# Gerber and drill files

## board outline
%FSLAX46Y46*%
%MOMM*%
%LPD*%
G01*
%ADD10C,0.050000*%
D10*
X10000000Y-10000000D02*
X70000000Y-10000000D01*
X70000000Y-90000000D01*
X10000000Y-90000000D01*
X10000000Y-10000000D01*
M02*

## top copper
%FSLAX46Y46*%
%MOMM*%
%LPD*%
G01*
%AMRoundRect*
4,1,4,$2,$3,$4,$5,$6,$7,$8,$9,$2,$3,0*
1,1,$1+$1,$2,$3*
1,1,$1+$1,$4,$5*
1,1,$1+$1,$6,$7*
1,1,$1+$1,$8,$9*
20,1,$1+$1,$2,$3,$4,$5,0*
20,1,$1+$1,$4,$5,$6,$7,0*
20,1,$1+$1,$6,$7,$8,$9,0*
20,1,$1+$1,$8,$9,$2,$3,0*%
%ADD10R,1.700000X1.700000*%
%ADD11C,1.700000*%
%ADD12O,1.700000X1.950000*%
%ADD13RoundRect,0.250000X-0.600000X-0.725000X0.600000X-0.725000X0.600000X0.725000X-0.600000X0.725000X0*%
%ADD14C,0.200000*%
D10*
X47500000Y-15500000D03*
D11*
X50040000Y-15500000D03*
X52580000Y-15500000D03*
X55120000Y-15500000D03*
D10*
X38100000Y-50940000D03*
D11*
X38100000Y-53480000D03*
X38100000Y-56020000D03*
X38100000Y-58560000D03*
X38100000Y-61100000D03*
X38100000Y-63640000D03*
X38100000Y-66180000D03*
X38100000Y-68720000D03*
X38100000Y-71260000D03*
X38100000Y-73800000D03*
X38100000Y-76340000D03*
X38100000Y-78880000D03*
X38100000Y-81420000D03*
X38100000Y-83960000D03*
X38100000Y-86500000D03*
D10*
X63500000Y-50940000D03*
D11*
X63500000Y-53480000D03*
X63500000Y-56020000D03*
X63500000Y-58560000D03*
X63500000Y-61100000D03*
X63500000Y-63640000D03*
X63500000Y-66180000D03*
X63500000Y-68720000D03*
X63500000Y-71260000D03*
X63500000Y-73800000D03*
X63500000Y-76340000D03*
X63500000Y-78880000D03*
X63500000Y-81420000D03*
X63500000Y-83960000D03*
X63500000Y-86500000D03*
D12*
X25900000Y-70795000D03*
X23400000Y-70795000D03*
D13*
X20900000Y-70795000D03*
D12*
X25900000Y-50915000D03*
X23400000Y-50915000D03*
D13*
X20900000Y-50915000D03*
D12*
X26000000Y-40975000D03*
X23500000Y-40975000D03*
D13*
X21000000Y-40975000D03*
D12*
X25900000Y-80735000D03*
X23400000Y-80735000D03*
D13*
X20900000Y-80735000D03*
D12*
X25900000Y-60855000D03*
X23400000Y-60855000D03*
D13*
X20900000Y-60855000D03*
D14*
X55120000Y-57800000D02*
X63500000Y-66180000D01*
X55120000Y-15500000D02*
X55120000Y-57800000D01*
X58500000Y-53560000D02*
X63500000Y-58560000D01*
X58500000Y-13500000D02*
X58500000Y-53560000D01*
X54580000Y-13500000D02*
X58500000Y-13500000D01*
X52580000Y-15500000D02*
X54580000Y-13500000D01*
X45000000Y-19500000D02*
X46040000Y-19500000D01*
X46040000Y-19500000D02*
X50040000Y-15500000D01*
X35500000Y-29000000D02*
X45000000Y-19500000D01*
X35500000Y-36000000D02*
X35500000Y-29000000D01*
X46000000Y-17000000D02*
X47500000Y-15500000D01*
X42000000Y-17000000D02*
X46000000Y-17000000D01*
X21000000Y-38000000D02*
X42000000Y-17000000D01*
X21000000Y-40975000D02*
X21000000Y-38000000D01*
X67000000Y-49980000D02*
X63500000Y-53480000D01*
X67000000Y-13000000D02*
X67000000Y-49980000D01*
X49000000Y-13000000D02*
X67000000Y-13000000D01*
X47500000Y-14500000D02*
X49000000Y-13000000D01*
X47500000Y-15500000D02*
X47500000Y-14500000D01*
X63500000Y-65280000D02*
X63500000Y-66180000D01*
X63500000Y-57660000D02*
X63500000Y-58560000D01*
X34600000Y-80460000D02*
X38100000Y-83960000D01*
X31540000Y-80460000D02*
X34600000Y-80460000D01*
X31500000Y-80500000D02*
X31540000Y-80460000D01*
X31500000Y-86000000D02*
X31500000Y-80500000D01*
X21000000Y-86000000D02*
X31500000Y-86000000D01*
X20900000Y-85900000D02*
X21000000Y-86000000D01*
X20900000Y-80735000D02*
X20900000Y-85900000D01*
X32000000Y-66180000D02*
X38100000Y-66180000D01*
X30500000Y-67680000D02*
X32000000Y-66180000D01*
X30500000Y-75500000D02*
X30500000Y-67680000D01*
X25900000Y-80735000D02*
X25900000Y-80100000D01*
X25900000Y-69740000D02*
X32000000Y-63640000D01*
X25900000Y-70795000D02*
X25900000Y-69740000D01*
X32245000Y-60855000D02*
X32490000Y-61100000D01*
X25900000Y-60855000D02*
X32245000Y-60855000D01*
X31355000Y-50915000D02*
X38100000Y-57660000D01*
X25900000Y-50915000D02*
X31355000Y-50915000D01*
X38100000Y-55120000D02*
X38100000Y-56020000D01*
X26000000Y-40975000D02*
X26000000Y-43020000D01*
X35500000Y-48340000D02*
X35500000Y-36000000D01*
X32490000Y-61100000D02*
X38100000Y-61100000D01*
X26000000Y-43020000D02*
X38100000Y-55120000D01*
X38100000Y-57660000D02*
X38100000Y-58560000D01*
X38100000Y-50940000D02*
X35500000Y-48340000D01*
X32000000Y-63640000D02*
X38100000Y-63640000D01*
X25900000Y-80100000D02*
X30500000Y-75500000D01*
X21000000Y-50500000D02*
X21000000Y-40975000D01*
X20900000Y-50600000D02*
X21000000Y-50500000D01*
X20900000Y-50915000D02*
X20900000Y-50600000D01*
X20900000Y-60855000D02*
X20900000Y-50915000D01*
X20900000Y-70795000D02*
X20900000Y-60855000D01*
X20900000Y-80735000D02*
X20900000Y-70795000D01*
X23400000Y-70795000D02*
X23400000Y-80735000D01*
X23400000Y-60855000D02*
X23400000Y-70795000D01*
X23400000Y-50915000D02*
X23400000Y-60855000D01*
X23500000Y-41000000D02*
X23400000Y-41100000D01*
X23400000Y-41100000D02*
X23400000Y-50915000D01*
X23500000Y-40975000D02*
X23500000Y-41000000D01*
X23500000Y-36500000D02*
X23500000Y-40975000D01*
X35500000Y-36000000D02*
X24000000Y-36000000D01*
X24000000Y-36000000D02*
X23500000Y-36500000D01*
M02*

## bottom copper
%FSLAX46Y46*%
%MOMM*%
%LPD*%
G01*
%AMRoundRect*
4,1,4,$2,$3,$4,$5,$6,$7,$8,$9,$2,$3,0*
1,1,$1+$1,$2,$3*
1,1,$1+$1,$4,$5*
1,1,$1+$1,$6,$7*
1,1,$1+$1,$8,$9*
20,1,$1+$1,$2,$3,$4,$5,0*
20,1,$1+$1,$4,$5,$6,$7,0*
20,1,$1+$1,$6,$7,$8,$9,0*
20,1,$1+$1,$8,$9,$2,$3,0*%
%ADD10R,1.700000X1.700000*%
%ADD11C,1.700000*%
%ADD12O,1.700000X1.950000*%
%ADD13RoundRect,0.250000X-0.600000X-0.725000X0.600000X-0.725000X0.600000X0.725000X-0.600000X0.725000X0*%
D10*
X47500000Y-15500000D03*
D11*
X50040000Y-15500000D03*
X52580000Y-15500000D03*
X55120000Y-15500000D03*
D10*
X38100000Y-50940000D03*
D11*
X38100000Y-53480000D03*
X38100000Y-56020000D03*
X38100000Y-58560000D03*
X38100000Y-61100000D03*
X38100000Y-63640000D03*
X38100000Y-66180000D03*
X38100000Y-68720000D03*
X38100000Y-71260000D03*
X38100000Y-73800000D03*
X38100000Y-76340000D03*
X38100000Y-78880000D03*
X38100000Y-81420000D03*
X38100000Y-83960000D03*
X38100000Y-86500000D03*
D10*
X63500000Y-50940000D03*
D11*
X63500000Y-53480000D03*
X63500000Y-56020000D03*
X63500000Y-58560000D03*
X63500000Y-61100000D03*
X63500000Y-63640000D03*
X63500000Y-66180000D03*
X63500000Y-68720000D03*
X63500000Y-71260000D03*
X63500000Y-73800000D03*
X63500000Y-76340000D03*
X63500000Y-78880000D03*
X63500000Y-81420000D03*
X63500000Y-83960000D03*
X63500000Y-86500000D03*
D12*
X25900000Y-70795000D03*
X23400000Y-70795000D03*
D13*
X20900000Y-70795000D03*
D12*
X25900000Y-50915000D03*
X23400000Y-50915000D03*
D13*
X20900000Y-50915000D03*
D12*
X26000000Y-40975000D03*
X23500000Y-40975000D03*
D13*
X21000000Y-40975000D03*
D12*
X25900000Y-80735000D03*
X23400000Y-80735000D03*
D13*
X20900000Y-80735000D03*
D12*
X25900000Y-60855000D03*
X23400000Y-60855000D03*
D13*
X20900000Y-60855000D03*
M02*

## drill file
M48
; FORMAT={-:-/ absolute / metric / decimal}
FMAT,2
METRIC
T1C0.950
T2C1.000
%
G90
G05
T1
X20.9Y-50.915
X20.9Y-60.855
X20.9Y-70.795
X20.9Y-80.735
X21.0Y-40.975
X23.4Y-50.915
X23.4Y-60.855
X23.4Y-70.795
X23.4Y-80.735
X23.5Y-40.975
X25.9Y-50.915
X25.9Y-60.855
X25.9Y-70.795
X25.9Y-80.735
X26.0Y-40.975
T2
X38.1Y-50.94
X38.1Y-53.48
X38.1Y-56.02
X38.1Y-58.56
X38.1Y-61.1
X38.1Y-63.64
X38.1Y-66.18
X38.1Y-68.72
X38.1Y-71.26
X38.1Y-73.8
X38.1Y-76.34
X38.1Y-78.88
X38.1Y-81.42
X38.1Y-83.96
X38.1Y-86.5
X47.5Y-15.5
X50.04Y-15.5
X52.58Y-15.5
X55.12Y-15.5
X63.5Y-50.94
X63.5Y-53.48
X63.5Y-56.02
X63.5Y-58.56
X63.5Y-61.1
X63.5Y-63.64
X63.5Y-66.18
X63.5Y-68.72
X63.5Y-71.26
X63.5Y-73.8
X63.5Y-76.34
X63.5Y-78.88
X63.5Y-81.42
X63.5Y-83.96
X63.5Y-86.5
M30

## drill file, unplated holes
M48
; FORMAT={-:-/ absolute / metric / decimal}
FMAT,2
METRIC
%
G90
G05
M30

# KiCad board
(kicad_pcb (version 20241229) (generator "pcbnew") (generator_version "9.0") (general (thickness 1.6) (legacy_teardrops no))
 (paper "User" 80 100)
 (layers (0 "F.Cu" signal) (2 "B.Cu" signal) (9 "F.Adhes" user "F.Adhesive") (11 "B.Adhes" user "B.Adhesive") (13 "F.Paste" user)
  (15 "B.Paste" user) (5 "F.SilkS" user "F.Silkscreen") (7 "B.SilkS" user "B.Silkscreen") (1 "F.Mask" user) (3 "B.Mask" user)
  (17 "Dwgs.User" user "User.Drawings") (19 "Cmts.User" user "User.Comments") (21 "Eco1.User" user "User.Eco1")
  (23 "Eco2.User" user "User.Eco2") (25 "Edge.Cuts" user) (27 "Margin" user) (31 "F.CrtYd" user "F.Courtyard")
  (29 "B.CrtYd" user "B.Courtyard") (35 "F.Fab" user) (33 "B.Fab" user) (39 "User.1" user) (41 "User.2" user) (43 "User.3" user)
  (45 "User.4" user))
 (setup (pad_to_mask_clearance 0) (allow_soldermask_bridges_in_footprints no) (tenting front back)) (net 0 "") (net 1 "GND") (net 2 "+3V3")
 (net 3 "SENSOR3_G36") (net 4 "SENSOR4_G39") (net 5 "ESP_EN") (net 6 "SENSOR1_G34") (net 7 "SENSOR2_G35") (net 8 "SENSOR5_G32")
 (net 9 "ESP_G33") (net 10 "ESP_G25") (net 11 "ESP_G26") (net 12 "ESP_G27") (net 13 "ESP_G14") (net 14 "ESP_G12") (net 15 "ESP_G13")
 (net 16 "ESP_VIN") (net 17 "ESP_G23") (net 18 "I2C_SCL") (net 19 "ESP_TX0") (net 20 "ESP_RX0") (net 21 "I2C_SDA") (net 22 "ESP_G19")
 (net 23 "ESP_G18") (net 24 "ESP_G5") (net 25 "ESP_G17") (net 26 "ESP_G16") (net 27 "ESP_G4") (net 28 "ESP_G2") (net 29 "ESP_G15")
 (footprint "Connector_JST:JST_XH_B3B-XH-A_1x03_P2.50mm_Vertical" (layer "F.Cu") (at 21 40.975)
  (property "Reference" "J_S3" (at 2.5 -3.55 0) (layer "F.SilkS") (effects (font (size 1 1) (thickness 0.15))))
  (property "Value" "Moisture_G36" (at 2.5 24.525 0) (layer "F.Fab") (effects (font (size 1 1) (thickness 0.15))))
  (pad "1" thru_hole roundrect (at 0 0) (size 1.7 1.95) (drill 0.95) (layers "*.Cu" "*.Mask") (remove_unused_layers no)
   (roundrect_rratio 0.147059) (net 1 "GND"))
  (pad "2" thru_hole oval (at 2.5 0) (size 1.7 1.95) (drill 0.95) (layers "*.Cu" "*.Mask") (remove_unused_layers no) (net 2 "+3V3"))
  (pad "3" thru_hole oval (at 5 0) (size 1.7 1.95) (drill 0.95) (layers "*.Cu" "*.Mask") (remove_unused_layers no) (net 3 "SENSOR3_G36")))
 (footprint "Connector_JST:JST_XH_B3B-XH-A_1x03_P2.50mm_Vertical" (layer "F.Cu") (at 20.9 50.915)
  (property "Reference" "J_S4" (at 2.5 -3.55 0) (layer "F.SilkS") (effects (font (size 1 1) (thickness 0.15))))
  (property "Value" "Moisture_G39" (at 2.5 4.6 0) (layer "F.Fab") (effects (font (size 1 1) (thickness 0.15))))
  (pad "1" thru_hole roundrect (at 0 0) (size 1.7 1.95) (drill 0.95) (layers "*.Cu" "*.Mask") (remove_unused_layers no)
   (roundrect_rratio 0.147059) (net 1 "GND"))
  (pad "2" thru_hole oval (at 2.5 0) (size 1.7 1.95) (drill 0.95) (layers "*.Cu" "*.Mask") (remove_unused_layers no) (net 2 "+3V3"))
  (pad "3" thru_hole oval (at 5 0) (size 1.7 1.95) (drill 0.95) (layers "*.Cu" "*.Mask") (remove_unused_layers no) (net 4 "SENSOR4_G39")))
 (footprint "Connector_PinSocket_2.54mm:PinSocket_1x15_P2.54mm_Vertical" (layer "F.Cu") (at 38.1 50.94)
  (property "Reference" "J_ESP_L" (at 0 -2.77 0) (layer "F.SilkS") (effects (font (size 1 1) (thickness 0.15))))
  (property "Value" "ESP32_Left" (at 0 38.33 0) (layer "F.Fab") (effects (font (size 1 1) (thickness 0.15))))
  (pad "1" thru_hole rect (at 0 0) (size 1.7 1.7) (drill 1) (layers "*.Cu" "*.Mask") (remove_unused_layers no) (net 2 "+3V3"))
  (pad "2" thru_hole circle (at 0 2.54) (size 1.7 1.7) (drill 1) (layers "*.Cu" "*.Mask") (remove_unused_layers no) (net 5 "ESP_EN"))
  (pad "3" thru_hole circle (at 0 5.08) (size 1.7 1.7) (drill 1) (layers "*.Cu" "*.Mask") (remove_unused_layers no) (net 3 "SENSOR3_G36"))
  (pad "4" thru_hole circle (at 0 7.62) (size 1.7 1.7) (drill 1) (layers "*.Cu" "*.Mask") (remove_unused_layers no) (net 4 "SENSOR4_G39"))
  (pad "5" thru_hole circle (at 0 10.16) (size 1.7 1.7) (drill 1) (layers "*.Cu" "*.Mask") (remove_unused_layers no) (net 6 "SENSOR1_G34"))
  (pad "6" thru_hole circle (at 0 12.7) (size 1.7 1.7) (drill 1) (layers "*.Cu" "*.Mask") (remove_unused_layers no) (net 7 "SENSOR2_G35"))
  (pad "7" thru_hole circle (at 0 15.24) (size 1.7 1.7) (drill 1) (layers "*.Cu" "*.Mask") (remove_unused_layers no) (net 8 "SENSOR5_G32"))
  (pad "8" thru_hole circle (at 0 17.78) (size 1.7 1.7) (drill 1) (layers "*.Cu" "*.Mask") (remove_unused_layers no) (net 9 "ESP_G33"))
  (pad "9" thru_hole circle (at 0 20.32) (size 1.7 1.7) (drill 1) (layers "*.Cu" "*.Mask") (remove_unused_layers no) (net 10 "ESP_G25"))
  (pad "10" thru_hole circle (at 0 22.86) (size 1.7 1.7) (drill 1) (layers "*.Cu" "*.Mask") (remove_unused_layers no) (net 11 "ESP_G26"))
  (pad "11" thru_hole circle (at 0 25.4) (size 1.7 1.7) (drill 1) (layers "*.Cu" "*.Mask") (remove_unused_layers no) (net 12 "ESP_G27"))
  (pad "12" thru_hole circle (at 0 27.94) (size 1.7 1.7) (drill 1) (layers "*.Cu" "*.Mask") (remove_unused_layers no) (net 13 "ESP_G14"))
  (pad "13" thru_hole circle (at 0 30.48) (size 1.7 1.7) (drill 1) (layers "*.Cu" "*.Mask") (remove_unused_layers no) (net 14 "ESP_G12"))
  (pad "14" thru_hole circle (at 0 33.02) (size 1.7 1.7) (drill 1) (layers "*.Cu" "*.Mask") (remove_unused_layers no) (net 1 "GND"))
  (pad "15" thru_hole circle (at 0 35.56) (size 1.7 1.7) (drill 1) (layers "*.Cu" "*.Mask") (remove_unused_layers no) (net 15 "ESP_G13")))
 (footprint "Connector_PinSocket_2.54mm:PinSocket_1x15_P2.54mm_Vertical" (layer "F.Cu") (at 63.5 50.94)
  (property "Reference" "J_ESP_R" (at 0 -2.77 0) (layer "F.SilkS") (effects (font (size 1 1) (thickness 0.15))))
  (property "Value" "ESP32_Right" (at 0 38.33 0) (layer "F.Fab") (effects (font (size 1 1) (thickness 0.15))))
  (pad "1" thru_hole rect (at 0 0) (size 1.7 1.7) (drill 1) (layers "*.Cu" "*.Mask") (remove_unused_layers no) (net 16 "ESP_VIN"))
  (pad "2" thru_hole circle (at 0 2.54) (size 1.7 1.7) (drill 1) (layers "*.Cu" "*.Mask") (remove_unused_layers no) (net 1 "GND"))
  (pad "3" thru_hole circle (at 0 5.08) (size 1.7 1.7) (drill 1) (layers "*.Cu" "*.Mask") (remove_unused_layers no) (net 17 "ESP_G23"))
  (pad "4" thru_hole circle (at 0 7.62) (size 1.7 1.7) (drill 1) (layers "*.Cu" "*.Mask") (remove_unused_layers no) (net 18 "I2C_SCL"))
  (pad "5" thru_hole circle (at 0 10.16) (size 1.7 1.7) (drill 1) (layers "*.Cu" "*.Mask") (remove_unused_layers no) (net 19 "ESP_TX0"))
  (pad "6" thru_hole circle (at 0 12.7) (size 1.7 1.7) (drill 1) (layers "*.Cu" "*.Mask") (remove_unused_layers no) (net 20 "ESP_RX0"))
  (pad "7" thru_hole circle (at 0 15.24) (size 1.7 1.7) (drill 1) (layers "*.Cu" "*.Mask") (remove_unused_layers no) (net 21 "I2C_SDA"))
  (pad "8" thru_hole circle (at 0 17.78) (size 1.7 1.7) (drill 1) (layers "*.Cu" "*.Mask") (remove_unused_layers no) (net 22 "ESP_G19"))
  (pad "9" thru_hole circle (at 0 20.32) (size 1.7 1.7) (drill 1) (layers "*.Cu" "*.Mask") (remove_unused_layers no) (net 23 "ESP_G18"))
  (pad "10" thru_hole circle (at 0 22.86) (size 1.7 1.7) (drill 1) (layers "*.Cu" "*.Mask") (remove_unused_layers no) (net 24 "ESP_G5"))
  (pad "11" thru_hole circle (at 0 25.4) (size 1.7 1.7) (drill 1) (layers "*.Cu" "*.Mask") (remove_unused_layers no) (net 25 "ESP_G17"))
  (pad "12" thru_hole circle (at 0 27.94) (size 1.7 1.7) (drill 1) (layers "*.Cu" "*.Mask") (remove_unused_layers no) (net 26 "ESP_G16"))
  (pad "13" thru_hole circle (at 0 30.48) (size 1.7 1.7) (drill 1) (layers "*.Cu" "*.Mask") (remove_unused_layers no) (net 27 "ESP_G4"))
  (pad "14" thru_hole circle (at 0 33.02) (size 1.7 1.7) (drill 1) (layers "*.Cu" "*.Mask") (remove_unused_layers no) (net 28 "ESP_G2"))
  (pad "15" thru_hole circle (at 0 35.56) (size 1.7 1.7) (drill 1) (layers "*.Cu" "*.Mask") (remove_unused_layers no) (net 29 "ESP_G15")))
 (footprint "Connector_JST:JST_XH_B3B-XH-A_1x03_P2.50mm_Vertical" (layer "F.Cu") (at 20.9 80.735)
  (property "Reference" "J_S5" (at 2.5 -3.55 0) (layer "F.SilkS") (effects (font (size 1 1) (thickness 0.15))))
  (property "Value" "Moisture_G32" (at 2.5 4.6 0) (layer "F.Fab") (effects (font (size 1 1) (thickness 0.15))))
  (pad "1" thru_hole roundrect (at 0 0) (size 1.7 1.95) (drill 0.95) (layers "*.Cu" "*.Mask") (remove_unused_layers no)
   (roundrect_rratio 0.147059) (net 1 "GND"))
  (pad "2" thru_hole oval (at 2.5 0) (size 1.7 1.95) (drill 0.95) (layers "*.Cu" "*.Mask") (remove_unused_layers no) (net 2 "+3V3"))
  (pad "3" thru_hole oval (at 5 0) (size 1.7 1.95) (drill 0.95) (layers "*.Cu" "*.Mask") (remove_unused_layers no) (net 8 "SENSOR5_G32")))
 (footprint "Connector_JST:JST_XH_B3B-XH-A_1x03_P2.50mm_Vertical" (layer "F.Cu") (at 20.9 60.855)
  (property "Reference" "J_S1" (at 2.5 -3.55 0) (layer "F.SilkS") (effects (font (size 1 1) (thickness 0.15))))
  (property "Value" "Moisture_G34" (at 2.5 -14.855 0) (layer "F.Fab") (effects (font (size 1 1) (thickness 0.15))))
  (pad "1" thru_hole roundrect (at 0 0) (size 1.7 1.95) (drill 0.95) (layers "*.Cu" "*.Mask") (remove_unused_layers no)
   (roundrect_rratio 0.147059) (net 1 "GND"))
  (pad "2" thru_hole oval (at 2.5 0) (size 1.7 1.95) (drill 0.95) (layers "*.Cu" "*.Mask") (remove_unused_layers no) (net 2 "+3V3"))
  (pad "3" thru_hole oval (at 5 0) (size 1.7 1.95) (drill 0.95) (layers "*.Cu" "*.Mask") (remove_unused_layers no) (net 6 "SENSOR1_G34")))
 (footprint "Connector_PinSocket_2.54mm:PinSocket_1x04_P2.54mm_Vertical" (layer "F.Cu") (at 47.5 15.5 90)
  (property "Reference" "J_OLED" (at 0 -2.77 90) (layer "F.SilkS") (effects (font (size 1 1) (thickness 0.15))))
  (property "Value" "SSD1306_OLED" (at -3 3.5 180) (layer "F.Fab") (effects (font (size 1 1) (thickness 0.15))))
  (pad "1" thru_hole rect (at 0 0 90) (size 1.7 1.7) (drill 1) (layers "*.Cu" "*.Mask") (remove_unused_layers no) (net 1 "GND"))
  (pad "2" thru_hole circle (at 0 2.54 90) (size 1.7 1.7) (drill 1) (layers "*.Cu" "*.Mask") (remove_unused_layers no) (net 2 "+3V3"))
  (pad "3" thru_hole circle (at 0 5.08 90) (size 1.7 1.7) (drill 1) (layers "*.Cu" "*.Mask") (remove_unused_layers no) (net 18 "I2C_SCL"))
  (pad "4" thru_hole circle (at 0 7.62 90) (size 1.7 1.7) (drill 1) (layers "*.Cu" "*.Mask") (remove_unused_layers no) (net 21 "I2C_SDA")))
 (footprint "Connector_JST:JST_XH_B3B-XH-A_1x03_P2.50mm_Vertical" (layer "F.Cu") (at 20.9 70.795)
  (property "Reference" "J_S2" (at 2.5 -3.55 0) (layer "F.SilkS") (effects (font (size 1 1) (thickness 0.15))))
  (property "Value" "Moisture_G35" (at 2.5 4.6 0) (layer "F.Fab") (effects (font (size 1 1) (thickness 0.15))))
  (pad "1" thru_hole roundrect (at 0 0) (size 1.7 1.95) (drill 0.95) (layers "*.Cu" "*.Mask") (remove_unused_layers no)
   (roundrect_rratio 0.147059) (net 1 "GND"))
  (pad "2" thru_hole oval (at 2.5 0) (size 1.7 1.95) (drill 0.95) (layers "*.Cu" "*.Mask") (remove_unused_layers no) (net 2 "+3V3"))
  (pad "3" thru_hole oval (at 5 0) (size 1.7 1.95) (drill 0.95) (layers "*.Cu" "*.Mask") (remove_unused_layers no) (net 7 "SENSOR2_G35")))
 (gr_rect (start 10 10) (end 70 90) (stroke (width 0.05) (type default)) (fill no) (layer "Edge.Cuts"))
 (segment (start 31.54 80.46) (end 34.6 80.46) (width 0.2) (layer "F.Cu") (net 1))
 (segment (start 20.9 85.9) (end 21 86) (width 0.2) (layer "F.Cu") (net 1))
 (segment (start 67 13) (end 67 49.98) (width 0.2) (layer "F.Cu") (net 1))
 (segment (start 67 49.98) (end 63.5 53.48) (width 0.2) (layer "F.Cu") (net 1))
 (segment (start 20.9 80.735) (end 20.9 85.9) (width 0.2) (layer "F.Cu") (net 1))
 (segment (start 21 40.975) (end 21 38) (width 0.2) (layer "F.Cu") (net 1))
 (segment (start 20.9 60.855) (end 20.9 50.915) (width 0.2) (layer "F.Cu") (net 1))
 (segment (start 20.9 50.6) (end 21 50.5) (width 0.2) (layer "F.Cu") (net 1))
 (segment (start 20.9 70.795) (end 20.9 60.855) (width 0.2) (layer "F.Cu") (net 1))
 (segment (start 31.5 80.5) (end 31.54 80.46) (width 0.2) (layer "F.Cu") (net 1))
 (segment (start 42 17) (end 46 17) (width 0.2) (layer "F.Cu") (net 1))
 (segment (start 31.5 86) (end 31.5 80.5) (width 0.2) (layer "F.Cu") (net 1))
 (segment (start 21 38) (end 42 17) (width 0.2) (layer "F.Cu") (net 1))
 (segment (start 21 50.5) (end 21 40.975) (width 0.2) (layer "F.Cu") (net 1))
 (segment (start 46 17) (end 47.5 15.5) (width 0.2) (layer "F.Cu") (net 1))
 (segment (start 20.9 80.735) (end 20.9 70.795) (width 0.2) (layer "F.Cu") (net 1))
 (segment (start 47.5 14.5) (end 49 13) (width 0.2) (layer "F.Cu") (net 1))
 (segment (start 49 13) (end 67 13) (width 0.2) (layer "F.Cu") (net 1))
 (segment (start 20.9 50.915) (end 20.9 50.6) (width 0.2) (layer "F.Cu") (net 1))
 (segment (start 47.5 15.5) (end 47.5 14.5) (width 0.2) (layer "F.Cu") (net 1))
 (segment (start 21 86) (end 31.5 86) (width 0.2) (layer "F.Cu") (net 1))
 (segment (start 34.6 80.46) (end 38.1 83.96) (width 0.2) (layer "F.Cu") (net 1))
 (segment (start 35.5 29) (end 45 19.5) (width 0.2) (layer "F.Cu") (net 2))
 (segment (start 23.5 36.5) (end 23.5 40.975) (width 0.2) (layer "F.Cu") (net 2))
 (segment (start 23.4 50.915) (end 23.4 60.855) (width 0.2) (layer "F.Cu") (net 2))
 (segment (start 23.4 60.855) (end 23.4 70.795) (width 0.2) (layer "F.Cu") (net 2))
 (segment (start 24 36) (end 23.5 36.5) (width 0.2) (layer "F.Cu") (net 2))
 (segment (start 23.5 40.975) (end 23.5 41) (width 0.2) (layer "F.Cu") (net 2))
 (segment (start 23.4 70.795) (end 23.4 80.735) (width 0.2) (layer "F.Cu") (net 2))
 (segment (start 23.4 41.1) (end 23.4 50.915) (width 0.2) (layer "F.Cu") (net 2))
 (segment (start 35.5 36) (end 35.5 29) (width 0.2) (layer "F.Cu") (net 2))
 (segment (start 35.5 48.34) (end 35.5 36) (width 0.2) (layer "F.Cu") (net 2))
 (segment (start 35.5 36) (end 24 36) (width 0.2) (layer "F.Cu") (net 2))
 (segment (start 45 19.5) (end 46.04 19.5) (width 0.2) (layer "F.Cu") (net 2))
 (segment (start 46.04 19.5) (end 50.04 15.5) (width 0.2) (layer "F.Cu") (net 2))
 (segment (start 38.1 50.94) (end 35.5 48.34) (width 0.2) (layer "F.Cu") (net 2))
 (segment (start 23.5 41) (end 23.4 41.1) (width 0.2) (layer "F.Cu") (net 2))
 (segment (start 31.355 50.915) (end 38.1 57.66) (width 0.2) (layer "F.Cu") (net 4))
 (segment (start 25.9 50.915) (end 31.355 50.915) (width 0.2) (layer "F.Cu") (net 4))
 (segment (start 38.1 57.66) (end 38.1 58.56) (width 0.2) (layer "F.Cu") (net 4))
 (segment (start 38.1 55.12) (end 38.1 56.02) (width 0.2) (layer "F.Cu") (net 3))
 (segment (start 26 43.02) (end 38.1 55.12) (width 0.2) (layer "F.Cu") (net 3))
 (segment (start 26 40.975) (end 26 43.02) (width 0.2) (layer "F.Cu") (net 3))
 (segment (start 25.9 80.1) (end 30.5 75.5) (width 0.2) (layer "F.Cu") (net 8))
 (segment (start 30.5 75.5) (end 30.5 67.68) (width 0.2) (layer "F.Cu") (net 8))
 (segment (start 25.9 80.735) (end 25.9 80.1) (width 0.2) (layer "F.Cu") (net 8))
 (segment (start 30.5 67.68) (end 32 66.18) (width 0.2) (layer "F.Cu") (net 8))
 (segment (start 32 66.18) (end 38.1 66.18) (width 0.2) (layer "F.Cu") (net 8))
 (segment (start 32.245 60.855) (end 32.49 61.1) (width 0.2) (layer "F.Cu") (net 6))
 (segment (start 32.49 61.1) (end 38.1 61.1) (width 0.2) (layer "F.Cu") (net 6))
 (segment (start 25.9 60.855) (end 32.245 60.855) (width 0.2) (layer "F.Cu") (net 6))
 (segment (start 25.9 70.795) (end 25.9 69.74) (width 0.2) (layer "F.Cu") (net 7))
 (segment (start 25.9 69.74) (end 32 63.64) (width 0.2) (layer "F.Cu") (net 7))
 (segment (start 32 63.64) (end 38.1 63.64) (width 0.2) (layer "F.Cu") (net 7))
 (segment (start 63.5 57.66) (end 63.5 58.56) (width 0.2) (layer "F.Cu") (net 18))
 (segment (start 58.5 53.56) (end 63.5 58.56) (width 0.2) (layer "F.Cu") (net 18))
 (segment (start 58.5 13.5) (end 58.5 53.56) (width 0.2) (layer "F.Cu") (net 18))
 (segment (start 52.58 15.5) (end 54.58 13.5) (width 0.2) (layer "F.Cu") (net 18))
 (segment (start 54.58 13.5) (end 58.5 13.5) (width 0.2) (layer "F.Cu") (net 18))
 (segment (start 55.12 15.5) (end 55.12 57.8) (width 0.2) (layer "F.Cu") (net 21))
 (segment (start 63.5 65.28) (end 63.5 66.18) (width 0.2) (layer "F.Cu") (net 21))
 (segment (start 55.12 57.8) (end 63.5 66.18) (width 0.2) (layer "F.Cu") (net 21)))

